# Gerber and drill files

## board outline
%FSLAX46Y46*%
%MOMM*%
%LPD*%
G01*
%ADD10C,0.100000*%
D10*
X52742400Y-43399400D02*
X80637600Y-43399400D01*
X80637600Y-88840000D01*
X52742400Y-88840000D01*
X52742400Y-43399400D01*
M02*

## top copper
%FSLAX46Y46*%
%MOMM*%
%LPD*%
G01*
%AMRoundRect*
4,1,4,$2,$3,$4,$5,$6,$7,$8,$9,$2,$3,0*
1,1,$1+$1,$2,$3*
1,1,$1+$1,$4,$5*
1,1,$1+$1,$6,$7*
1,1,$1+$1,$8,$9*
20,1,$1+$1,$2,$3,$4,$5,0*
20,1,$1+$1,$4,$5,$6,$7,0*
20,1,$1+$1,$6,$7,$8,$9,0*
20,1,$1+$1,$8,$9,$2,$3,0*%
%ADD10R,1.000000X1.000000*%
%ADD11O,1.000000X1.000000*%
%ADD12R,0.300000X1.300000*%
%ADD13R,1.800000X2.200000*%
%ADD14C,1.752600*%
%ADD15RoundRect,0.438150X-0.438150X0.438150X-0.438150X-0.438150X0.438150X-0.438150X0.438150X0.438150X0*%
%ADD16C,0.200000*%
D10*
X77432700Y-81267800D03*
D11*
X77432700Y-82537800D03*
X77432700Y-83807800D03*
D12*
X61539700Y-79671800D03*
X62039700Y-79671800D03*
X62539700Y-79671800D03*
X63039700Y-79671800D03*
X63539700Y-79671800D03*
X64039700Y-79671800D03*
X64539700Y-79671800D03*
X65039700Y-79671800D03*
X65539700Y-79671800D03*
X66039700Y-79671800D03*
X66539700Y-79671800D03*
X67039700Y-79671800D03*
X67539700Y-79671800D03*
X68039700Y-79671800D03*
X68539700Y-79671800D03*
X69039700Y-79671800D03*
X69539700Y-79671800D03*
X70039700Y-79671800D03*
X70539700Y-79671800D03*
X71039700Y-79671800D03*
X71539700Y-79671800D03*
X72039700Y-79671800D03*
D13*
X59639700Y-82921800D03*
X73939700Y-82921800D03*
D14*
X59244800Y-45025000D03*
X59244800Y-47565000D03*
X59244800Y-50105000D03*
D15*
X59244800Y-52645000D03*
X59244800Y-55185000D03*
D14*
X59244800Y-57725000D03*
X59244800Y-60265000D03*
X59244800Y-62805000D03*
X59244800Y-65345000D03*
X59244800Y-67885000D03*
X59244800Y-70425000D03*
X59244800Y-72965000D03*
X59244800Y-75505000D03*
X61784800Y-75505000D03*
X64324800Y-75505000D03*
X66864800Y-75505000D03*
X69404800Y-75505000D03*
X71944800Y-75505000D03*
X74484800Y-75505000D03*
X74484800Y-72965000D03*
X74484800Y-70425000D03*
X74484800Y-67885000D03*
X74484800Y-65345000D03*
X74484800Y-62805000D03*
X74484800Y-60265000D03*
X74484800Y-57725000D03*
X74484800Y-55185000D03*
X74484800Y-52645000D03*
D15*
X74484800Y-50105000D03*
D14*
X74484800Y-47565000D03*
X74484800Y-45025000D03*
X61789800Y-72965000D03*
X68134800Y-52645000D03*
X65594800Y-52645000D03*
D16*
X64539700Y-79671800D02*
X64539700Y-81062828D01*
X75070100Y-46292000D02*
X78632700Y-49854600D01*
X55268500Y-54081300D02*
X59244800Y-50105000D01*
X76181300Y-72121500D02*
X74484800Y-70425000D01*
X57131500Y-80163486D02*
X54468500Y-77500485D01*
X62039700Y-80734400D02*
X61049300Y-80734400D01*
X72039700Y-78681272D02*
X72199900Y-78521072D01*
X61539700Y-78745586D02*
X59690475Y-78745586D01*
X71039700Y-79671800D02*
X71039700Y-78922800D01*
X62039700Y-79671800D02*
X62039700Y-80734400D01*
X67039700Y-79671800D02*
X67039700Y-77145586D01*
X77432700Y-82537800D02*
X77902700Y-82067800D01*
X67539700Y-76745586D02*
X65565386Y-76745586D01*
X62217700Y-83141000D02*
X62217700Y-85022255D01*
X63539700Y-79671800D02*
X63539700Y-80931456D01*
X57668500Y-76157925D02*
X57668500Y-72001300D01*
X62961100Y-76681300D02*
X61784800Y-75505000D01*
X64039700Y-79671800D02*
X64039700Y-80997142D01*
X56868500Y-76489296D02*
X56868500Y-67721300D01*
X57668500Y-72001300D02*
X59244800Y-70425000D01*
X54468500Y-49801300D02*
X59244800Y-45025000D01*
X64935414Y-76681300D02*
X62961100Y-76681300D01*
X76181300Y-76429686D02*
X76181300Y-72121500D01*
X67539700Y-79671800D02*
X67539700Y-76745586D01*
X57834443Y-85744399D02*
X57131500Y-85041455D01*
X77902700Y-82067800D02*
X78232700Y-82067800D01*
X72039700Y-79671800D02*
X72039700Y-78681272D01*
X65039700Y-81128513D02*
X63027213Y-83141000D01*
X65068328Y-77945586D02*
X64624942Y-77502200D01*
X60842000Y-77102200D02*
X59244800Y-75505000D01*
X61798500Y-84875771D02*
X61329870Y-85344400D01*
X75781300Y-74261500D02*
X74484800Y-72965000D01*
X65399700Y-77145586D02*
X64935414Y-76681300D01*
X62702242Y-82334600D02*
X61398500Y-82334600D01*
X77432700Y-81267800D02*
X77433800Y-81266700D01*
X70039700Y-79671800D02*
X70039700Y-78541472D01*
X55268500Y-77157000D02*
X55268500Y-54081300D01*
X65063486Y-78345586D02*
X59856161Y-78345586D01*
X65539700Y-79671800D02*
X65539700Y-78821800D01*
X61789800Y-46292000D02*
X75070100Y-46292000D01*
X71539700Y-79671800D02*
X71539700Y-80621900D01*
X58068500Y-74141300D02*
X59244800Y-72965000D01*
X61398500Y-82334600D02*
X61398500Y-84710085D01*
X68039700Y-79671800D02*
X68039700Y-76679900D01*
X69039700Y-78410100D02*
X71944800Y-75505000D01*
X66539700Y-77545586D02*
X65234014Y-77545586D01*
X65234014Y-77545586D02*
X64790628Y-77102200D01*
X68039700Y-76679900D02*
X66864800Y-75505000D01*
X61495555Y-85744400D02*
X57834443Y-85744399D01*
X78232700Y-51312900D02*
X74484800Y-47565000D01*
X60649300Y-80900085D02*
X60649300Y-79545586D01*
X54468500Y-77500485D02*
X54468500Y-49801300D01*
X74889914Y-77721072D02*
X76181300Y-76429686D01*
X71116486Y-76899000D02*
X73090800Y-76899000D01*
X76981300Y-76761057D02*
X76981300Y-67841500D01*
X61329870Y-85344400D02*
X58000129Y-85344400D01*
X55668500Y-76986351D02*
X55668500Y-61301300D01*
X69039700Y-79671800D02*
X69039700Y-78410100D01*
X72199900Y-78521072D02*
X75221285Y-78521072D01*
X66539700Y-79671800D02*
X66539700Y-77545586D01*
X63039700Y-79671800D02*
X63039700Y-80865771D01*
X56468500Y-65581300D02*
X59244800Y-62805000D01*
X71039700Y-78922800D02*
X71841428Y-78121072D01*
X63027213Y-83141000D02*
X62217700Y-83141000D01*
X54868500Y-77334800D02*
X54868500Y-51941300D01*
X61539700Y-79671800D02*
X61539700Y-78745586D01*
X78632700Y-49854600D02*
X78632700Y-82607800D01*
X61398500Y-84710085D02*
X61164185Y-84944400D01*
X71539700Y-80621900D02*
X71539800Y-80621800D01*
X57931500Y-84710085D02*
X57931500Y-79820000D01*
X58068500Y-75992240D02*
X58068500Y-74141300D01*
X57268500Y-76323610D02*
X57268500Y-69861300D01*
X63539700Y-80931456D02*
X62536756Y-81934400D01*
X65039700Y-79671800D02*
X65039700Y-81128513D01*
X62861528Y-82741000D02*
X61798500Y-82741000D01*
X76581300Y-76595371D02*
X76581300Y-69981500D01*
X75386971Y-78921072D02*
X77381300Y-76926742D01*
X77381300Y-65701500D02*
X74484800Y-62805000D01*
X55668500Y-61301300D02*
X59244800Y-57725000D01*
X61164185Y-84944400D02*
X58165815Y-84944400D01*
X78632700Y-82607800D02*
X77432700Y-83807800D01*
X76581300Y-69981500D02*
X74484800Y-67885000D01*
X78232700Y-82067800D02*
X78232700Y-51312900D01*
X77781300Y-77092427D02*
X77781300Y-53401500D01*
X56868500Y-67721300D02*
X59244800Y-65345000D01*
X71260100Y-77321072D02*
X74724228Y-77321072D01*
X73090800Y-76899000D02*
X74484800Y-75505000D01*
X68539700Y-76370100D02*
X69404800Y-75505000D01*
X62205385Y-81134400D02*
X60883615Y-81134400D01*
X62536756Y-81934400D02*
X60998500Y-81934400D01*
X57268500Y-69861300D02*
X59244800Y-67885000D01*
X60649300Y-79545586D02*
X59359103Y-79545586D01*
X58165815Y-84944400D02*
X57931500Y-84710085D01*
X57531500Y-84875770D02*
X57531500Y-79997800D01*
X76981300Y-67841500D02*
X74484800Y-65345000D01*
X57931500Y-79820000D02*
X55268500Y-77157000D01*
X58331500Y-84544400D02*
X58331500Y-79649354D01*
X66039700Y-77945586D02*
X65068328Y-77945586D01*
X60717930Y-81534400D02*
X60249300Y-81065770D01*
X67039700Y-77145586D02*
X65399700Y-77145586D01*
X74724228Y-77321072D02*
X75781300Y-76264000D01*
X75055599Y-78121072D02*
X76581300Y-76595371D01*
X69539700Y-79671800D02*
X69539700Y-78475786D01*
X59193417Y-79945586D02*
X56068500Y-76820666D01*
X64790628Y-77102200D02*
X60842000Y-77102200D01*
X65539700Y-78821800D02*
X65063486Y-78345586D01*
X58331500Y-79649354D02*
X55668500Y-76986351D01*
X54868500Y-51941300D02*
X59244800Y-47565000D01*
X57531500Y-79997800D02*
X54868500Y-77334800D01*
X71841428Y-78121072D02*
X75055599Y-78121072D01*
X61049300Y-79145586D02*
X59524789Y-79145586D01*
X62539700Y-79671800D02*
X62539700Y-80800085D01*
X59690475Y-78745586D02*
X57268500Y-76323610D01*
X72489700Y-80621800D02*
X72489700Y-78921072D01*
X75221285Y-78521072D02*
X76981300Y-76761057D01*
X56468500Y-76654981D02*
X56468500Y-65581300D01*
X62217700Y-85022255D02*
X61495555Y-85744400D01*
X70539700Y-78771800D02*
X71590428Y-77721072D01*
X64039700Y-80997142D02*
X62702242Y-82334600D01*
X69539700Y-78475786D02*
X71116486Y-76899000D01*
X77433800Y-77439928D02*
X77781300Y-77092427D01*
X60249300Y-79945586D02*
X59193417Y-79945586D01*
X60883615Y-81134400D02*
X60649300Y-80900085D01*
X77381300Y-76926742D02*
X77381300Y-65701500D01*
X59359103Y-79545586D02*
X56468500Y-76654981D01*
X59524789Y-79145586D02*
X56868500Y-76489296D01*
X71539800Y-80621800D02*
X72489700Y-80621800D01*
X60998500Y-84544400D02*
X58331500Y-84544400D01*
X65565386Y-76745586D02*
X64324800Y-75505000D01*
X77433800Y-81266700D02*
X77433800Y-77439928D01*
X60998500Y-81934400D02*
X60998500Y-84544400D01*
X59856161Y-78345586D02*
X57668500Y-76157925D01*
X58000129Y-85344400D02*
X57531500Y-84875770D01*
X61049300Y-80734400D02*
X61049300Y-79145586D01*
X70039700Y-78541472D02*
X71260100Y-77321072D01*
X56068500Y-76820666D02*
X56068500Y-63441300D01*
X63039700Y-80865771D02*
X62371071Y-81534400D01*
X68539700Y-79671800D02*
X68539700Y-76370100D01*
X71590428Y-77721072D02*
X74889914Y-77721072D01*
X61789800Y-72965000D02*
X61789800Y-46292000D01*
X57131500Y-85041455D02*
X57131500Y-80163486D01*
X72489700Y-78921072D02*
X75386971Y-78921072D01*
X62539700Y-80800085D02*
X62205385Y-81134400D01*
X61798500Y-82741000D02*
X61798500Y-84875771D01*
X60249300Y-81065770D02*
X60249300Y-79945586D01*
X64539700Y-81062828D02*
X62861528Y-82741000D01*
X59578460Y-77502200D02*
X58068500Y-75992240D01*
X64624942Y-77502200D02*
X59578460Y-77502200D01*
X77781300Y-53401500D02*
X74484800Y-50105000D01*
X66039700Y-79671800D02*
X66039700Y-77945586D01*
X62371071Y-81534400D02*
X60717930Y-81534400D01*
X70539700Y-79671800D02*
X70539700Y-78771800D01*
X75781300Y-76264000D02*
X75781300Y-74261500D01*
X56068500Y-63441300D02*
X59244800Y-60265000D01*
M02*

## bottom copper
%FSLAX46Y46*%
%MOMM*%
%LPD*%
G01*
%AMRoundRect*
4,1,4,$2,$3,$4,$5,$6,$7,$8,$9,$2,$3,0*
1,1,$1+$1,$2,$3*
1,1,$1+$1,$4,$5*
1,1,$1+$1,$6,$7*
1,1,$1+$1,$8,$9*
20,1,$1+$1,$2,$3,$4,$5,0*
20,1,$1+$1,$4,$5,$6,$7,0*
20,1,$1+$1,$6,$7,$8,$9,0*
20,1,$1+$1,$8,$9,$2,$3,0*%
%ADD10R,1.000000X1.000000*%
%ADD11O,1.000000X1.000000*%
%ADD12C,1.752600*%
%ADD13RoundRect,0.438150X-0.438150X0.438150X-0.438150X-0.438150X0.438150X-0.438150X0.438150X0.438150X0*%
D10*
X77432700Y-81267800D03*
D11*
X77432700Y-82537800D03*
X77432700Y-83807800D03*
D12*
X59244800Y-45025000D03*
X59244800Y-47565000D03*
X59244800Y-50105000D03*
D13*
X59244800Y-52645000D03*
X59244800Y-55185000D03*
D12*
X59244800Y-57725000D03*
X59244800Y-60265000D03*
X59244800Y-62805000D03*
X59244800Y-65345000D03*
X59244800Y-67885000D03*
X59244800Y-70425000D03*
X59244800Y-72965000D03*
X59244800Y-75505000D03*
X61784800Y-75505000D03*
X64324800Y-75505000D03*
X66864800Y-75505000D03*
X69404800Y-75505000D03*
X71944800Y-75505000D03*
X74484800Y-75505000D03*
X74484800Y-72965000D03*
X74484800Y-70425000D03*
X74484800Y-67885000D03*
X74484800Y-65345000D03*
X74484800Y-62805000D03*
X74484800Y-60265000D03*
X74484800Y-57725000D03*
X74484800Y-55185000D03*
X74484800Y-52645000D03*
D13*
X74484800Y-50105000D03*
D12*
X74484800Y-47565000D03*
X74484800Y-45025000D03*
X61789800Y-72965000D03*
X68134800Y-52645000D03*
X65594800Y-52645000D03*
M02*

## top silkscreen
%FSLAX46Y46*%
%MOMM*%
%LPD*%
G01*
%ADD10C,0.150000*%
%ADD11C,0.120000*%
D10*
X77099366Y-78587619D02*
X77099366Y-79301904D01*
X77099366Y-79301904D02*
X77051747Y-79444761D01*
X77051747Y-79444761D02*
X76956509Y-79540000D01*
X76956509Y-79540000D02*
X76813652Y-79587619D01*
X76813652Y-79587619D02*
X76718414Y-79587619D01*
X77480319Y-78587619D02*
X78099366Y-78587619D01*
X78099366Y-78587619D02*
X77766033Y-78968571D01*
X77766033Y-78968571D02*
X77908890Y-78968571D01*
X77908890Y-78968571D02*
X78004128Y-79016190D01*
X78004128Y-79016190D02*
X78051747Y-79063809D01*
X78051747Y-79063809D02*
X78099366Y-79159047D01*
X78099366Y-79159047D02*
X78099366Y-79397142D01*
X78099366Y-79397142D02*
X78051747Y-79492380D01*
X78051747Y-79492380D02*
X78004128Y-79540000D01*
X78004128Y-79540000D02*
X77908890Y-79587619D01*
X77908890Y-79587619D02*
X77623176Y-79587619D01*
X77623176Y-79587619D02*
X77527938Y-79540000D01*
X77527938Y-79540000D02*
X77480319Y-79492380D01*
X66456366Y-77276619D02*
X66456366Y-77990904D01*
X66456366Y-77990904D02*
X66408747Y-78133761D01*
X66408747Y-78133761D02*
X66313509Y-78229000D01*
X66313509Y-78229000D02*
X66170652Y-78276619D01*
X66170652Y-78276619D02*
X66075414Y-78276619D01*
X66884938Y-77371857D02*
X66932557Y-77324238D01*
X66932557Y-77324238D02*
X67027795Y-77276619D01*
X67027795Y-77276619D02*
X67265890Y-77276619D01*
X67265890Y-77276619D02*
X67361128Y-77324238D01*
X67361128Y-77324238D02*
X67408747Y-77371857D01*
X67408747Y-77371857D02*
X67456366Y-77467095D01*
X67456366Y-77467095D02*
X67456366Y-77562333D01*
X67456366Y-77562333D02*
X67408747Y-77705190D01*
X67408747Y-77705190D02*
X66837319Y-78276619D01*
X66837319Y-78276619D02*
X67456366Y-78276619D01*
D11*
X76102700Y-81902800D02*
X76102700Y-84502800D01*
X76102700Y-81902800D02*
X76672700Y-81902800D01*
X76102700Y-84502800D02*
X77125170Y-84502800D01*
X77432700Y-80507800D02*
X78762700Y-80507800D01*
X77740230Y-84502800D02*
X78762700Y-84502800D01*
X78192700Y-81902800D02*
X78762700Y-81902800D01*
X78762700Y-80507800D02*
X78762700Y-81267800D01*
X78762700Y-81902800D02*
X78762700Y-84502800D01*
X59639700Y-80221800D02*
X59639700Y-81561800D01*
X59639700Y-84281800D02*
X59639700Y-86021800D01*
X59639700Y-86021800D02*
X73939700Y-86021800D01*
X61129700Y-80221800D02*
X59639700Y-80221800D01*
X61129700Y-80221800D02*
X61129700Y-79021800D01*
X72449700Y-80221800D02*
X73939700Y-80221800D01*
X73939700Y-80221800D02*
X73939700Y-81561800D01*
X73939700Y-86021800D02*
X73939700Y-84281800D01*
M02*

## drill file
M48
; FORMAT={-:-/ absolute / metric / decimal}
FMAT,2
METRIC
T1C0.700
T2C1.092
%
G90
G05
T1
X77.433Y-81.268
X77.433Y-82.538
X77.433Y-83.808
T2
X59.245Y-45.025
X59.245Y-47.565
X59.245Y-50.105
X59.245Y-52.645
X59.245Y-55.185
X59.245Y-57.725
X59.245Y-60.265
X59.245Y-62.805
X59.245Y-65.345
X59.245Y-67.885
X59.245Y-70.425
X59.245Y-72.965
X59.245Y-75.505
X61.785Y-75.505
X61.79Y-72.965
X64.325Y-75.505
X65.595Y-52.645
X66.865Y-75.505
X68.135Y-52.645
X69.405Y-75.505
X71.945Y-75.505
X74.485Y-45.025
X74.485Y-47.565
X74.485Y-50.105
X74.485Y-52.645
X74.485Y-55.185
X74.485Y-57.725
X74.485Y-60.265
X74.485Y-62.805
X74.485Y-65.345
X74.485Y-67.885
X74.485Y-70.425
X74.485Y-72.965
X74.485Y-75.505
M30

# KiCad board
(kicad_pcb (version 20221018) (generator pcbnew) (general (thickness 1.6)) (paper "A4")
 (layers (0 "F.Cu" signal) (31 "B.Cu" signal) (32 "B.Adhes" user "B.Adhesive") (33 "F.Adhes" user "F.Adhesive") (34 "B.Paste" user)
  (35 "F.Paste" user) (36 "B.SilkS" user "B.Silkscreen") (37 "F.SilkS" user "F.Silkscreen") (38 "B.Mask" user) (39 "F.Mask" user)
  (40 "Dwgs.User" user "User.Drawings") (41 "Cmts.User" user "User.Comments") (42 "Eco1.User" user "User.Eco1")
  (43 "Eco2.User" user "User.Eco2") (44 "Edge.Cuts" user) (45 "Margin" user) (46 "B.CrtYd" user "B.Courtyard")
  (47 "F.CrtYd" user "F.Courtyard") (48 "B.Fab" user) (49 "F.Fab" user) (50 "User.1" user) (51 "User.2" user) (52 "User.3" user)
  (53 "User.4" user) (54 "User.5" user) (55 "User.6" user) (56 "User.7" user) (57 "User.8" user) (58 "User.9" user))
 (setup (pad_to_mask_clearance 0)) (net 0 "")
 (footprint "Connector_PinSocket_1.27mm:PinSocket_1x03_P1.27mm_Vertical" (layer "F.Cu") (at 77.4327 81.2678)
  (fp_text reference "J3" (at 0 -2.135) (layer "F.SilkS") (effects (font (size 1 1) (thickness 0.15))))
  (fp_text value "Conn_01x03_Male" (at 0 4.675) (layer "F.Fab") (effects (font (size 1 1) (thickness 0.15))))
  (fp_line (start -1.33 0.635) (end -1.33 3.235) (stroke (width 0.12) (type solid)) (layer "F.SilkS"))
  (fp_line (start -1.33 0.635) (end -0.76 0.635) (stroke (width 0.12) (type solid)) (layer "F.SilkS"))
  (fp_line (start -1.33 3.235) (end -0.30753 3.235) (stroke (width 0.12) (type solid)) (layer "F.SilkS"))
  (fp_line (start 0 -0.76) (end 1.33 -0.76) (stroke (width 0.12) (type solid)) (layer "F.SilkS"))
  (fp_line (start 0.30753 3.235) (end 1.33 3.235) (stroke (width 0.12) (type solid)) (layer "F.SilkS"))
  (fp_line (start 0.76 0.635) (end 1.33 0.635) (stroke (width 0.12) (type solid)) (layer "F.SilkS"))
  (fp_line (start 1.33 -0.76) (end 1.33 0) (stroke (width 0.12) (type solid)) (layer "F.SilkS"))
  (fp_line (start 1.33 0.635) (end 1.33 3.235) (stroke (width 0.12) (type solid)) (layer "F.SilkS"))
  (pad "1" thru_hole rect (at 0 0) (size 1 1) (drill 0.7) (layers "*.Cu" "*.Mask"))
  (pad "2" thru_hole oval (at 0 1.27) (size 1 1) (drill 0.7) (layers "*.Cu" "*.Mask"))
  (pad "3" thru_hole oval (at 0 2.54) (size 1 1) (drill 0.7) (layers "*.Cu" "*.Mask")))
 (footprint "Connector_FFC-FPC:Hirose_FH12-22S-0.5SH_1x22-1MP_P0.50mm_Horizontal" (layer "F.Cu") (at 66.7897 81.5218)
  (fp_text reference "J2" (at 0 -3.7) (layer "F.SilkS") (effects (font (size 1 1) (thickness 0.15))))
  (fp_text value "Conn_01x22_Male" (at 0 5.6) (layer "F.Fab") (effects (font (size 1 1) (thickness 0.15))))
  (fp_line (start -7.15 -1.3) (end -7.15 0.04) (stroke (width 0.12) (type solid)) (layer "F.SilkS"))
  (fp_line (start -7.15 2.76) (end -7.15 4.5) (stroke (width 0.12) (type solid)) (layer "F.SilkS"))
  (fp_line (start -7.15 4.5) (end 7.15 4.5) (stroke (width 0.12) (type solid)) (layer "F.SilkS"))
  (fp_line (start -5.66 -1.3) (end -7.15 -1.3) (stroke (width 0.12) (type solid)) (layer "F.SilkS"))
  (fp_line (start -5.66 -1.3) (end -5.66 -2.5) (stroke (width 0.12) (type solid)) (layer "F.SilkS"))
  (fp_line (start 5.66 -1.3) (end 7.15 -1.3) (stroke (width 0.12) (type solid)) (layer "F.SilkS"))
  (fp_line (start 7.15 -1.3) (end 7.15 0.04) (stroke (width 0.12) (type solid)) (layer "F.SilkS"))
  (fp_line (start 7.15 4.5) (end 7.15 2.76) (stroke (width 0.12) (type solid)) (layer "F.SilkS"))
  (pad "1" smd rect (at -5.25 -1.85) (size 0.3 1.3) (layers "F.Cu" "F.Paste" "F.Mask"))
  (pad "2" smd rect (at -4.75 -1.85) (size 0.3 1.3) (layers "F.Cu" "F.Paste" "F.Mask"))
  (pad "3" smd rect (at -4.25 -1.85) (size 0.3 1.3) (layers "F.Cu" "F.Paste" "F.Mask"))
  (pad "4" smd rect (at -3.75 -1.85) (size 0.3 1.3) (layers "F.Cu" "F.Paste" "F.Mask"))
  (pad "5" smd rect (at -3.25 -1.85) (size 0.3 1.3) (layers "F.Cu" "F.Paste" "F.Mask"))
  (pad "6" smd rect (at -2.75 -1.85) (size 0.3 1.3) (layers "F.Cu" "F.Paste" "F.Mask"))
  (pad "7" smd rect (at -2.25 -1.85) (size 0.3 1.3) (layers "F.Cu" "F.Paste" "F.Mask"))
  (pad "8" smd rect (at -1.75 -1.85) (size 0.3 1.3) (layers "F.Cu" "F.Paste" "F.Mask"))
  (pad "9" smd rect (at -1.25 -1.85) (size 0.3 1.3) (layers "F.Cu" "F.Paste" "F.Mask"))
  (pad "10" smd rect (at -0.75 -1.85) (size 0.3 1.3) (layers "F.Cu" "F.Paste" "F.Mask"))
  (pad "11" smd rect (at -0.25 -1.85) (size 0.3 1.3) (layers "F.Cu" "F.Paste" "F.Mask"))
  (pad "12" smd rect (at 0.25 -1.85) (size 0.3 1.3) (layers "F.Cu" "F.Paste" "F.Mask"))
  (pad "13" smd rect (at 0.75 -1.85) (size 0.3 1.3) (layers "F.Cu" "F.Paste" "F.Mask"))
  (pad "14" smd rect (at 1.25 -1.85) (size 0.3 1.3) (layers "F.Cu" "F.Paste" "F.Mask"))
  (pad "15" smd rect (at 1.75 -1.85) (size 0.3 1.3) (layers "F.Cu" "F.Paste" "F.Mask"))
  (pad "16" smd rect (at 2.25 -1.85) (size 0.3 1.3) (layers "F.Cu" "F.Paste" "F.Mask"))
  (pad "17" smd rect (at 2.75 -1.85) (size 0.3 1.3) (layers "F.Cu" "F.Paste" "F.Mask"))
  (pad "18" smd rect (at 3.25 -1.85) (size 0.3 1.3) (layers "F.Cu" "F.Paste" "F.Mask"))
  (pad "19" smd rect (at 3.75 -1.85) (size 0.3 1.3) (layers "F.Cu" "F.Paste" "F.Mask"))
  (pad "20" smd rect (at 4.25 -1.85) (size 0.3 1.3) (layers "F.Cu" "F.Paste" "F.Mask"))
  (pad "21" smd rect (at 4.75 -1.85) (size 0.3 1.3) (layers "F.Cu" "F.Paste" "F.Mask"))
  (pad "22" smd rect (at 5.25 -1.85) (size 0.3 1.3) (layers "F.Cu" "F.Paste" "F.Mask"))
  (pad "MP" smd rect (at -7.15 1.4) (size 1.8 2.2) (layers "F.Cu" "F.Paste" "F.Mask"))
  (pad "MP" smd rect (at 7.15 1.4) (size 1.8 2.2) (layers "F.Cu" "F.Paste" "F.Mask")))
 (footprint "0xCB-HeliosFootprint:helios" (layer "F.Cu") (at 66.8648 61.535)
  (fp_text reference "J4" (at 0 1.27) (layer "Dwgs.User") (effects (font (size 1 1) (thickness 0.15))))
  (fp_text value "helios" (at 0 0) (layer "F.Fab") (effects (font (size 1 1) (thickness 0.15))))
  (pad "1" thru_hole circle (at -7.62 -16.51 270) (size 1.7526 1.7526) (drill 1.0922) (layers "*.Cu" "*.Mask"))
  (pad "2" thru_hole circle (at -7.62 -13.97 270) (size 1.7526 1.7526) (drill 1.0922) (layers "*.Cu" "*.Mask"))
  (pad "3" thru_hole circle (at -7.62 -11.43 270) (size 1.7526 1.7526) (drill 1.0922) (layers "*.Cu" "*.Mask"))
  (pad "4" thru_hole roundrect (at -7.62 -8.89 270) (size 1.7526 1.7526) (drill 1.0922) (layers "*.Cu" "*.Mask") (roundrect_rratio 0.25))
  (pad "5" thru_hole roundrect (at -7.62 -6.35 270) (size 1.7526 1.7526) (drill 1.0922) (layers "*.Cu" "*.Mask") (roundrect_rratio 0.25))
  (pad "6" thru_hole circle (at -7.62 -3.81 270) (size 1.7526 1.7526) (drill 1.0922) (layers "*.Cu" "*.Mask"))
  (pad "7" thru_hole circle (at -7.62 -1.27 270) (size 1.7526 1.7526) (drill 1.0922) (layers "*.Cu" "*.Mask"))
  (pad "8" thru_hole circle (at -7.62 1.27 270) (size 1.7526 1.7526) (drill 1.0922) (layers "*.Cu" "*.Mask"))
  (pad "9" thru_hole circle (at -7.62 3.81 270) (size 1.7526 1.7526) (drill 1.0922) (layers "*.Cu" "*.Mask"))
  (pad "10" thru_hole circle (at -7.62 6.35 270) (size 1.7526 1.7526) (drill 1.0922) (layers "*.Cu" "*.Mask"))
  (pad "11" thru_hole circle (at -7.62 8.89 270) (size 1.7526 1.7526) (drill 1.0922) (layers "*.Cu" "*.Mask"))
  (pad "12" thru_hole circle (at -7.62 11.43 270) (size 1.7526 1.7526) (drill 1.0922) (layers "*.Cu" "*.Mask"))
  (pad "13" thru_hole circle (at -7.62 13.97 270) (size 1.7526 1.7526) (drill 1.0922) (layers "*.Cu" "*.Mask"))
  (pad "14" thru_hole circle (at -5.08 13.97 270) (size 1.7526 1.7526) (drill 1.0922) (layers "*.Cu" "*.Mask"))
  (pad "15" thru_hole circle (at -2.54 13.97 270) (size 1.7526 1.7526) (drill 1.0922) (layers "*.Cu" "*.Mask"))
  (pad "16" thru_hole circle (at 0 13.97 270) (size 1.7526 1.7526) (drill 1.0922) (layers "*.Cu" "*.Mask"))
  (pad "17" thru_hole circle (at 2.54 13.97 270) (size 1.7526 1.7526) (drill 1.0922) (layers "*.Cu" "*.Mask"))
  (pad "18" thru_hole circle (at 5.08 13.97 270) (size 1.7526 1.7526) (drill 1.0922) (layers "*.Cu" "*.Mask"))
  (pad "19" thru_hole circle (at 7.62 13.97 270) (size 1.7526 1.7526) (drill 1.0922) (layers "*.Cu" "*.Mask"))
  (pad "20" thru_hole circle (at 7.62 11.43 270) (size 1.7526 1.7526) (drill 1.0922) (layers "*.Cu" "*.Mask"))
  (pad "21" thru_hole circle (at 7.62 8.89 270) (size 1.7526 1.7526) (drill 1.0922) (layers "*.Cu" "*.Mask"))
  (pad "22" thru_hole circle (at 7.62 6.35 270) (size 1.7526 1.7526) (drill 1.0922) (layers "*.Cu" "*.Mask"))
  (pad "23" thru_hole circle (at 7.62 3.81 270) (size 1.7526 1.7526) (drill 1.0922) (layers "*.Cu" "*.Mask"))
  (pad "24" thru_hole circle (at 7.62 1.27 270) (size 1.7526 1.7526) (drill 1.0922) (layers "*.Cu" "*.Mask"))
  (pad "25" thru_hole circle (at 7.62 -1.27 270) (size 1.7526 1.7526) (drill 1.0922) (layers "*.Cu" "*.Mask"))
  (pad "26" thru_hole circle (at 7.62 -3.81 270) (size 1.7526 1.7526) (drill 1.0922) (layers "*.Cu" "*.Mask"))
  (pad "27" thru_hole circle (at 7.62 -6.35 270) (size 1.7526 1.7526) (drill 1.0922) (layers "*.Cu" "*.Mask"))
  (pad "28" thru_hole circle (at 7.62 -8.89 270) (size 1.7526 1.7526) (drill 1.0922) (layers "*.Cu" "*.Mask"))
  (pad "29" thru_hole roundrect (at 7.62 -11.43 270) (size 1.7526 1.7526) (drill 1.0922) (layers "*.Cu" "*.Mask") (roundrect_rratio 0.25))
  (pad "30" thru_hole circle (at 7.62 -13.97 270) (size 1.7526 1.7526) (drill 1.0922) (layers "*.Cu" "*.Mask"))
  (pad "31" thru_hole circle (at 7.62 -16.51 270) (size 1.7526 1.7526) (drill 1.0922) (layers "*.Cu" "*.Mask"))
  (pad "32" thru_hole circle (at -5.075 11.43 270) (size 1.7526 1.7526) (drill 1.0922) (layers "*.Cu" "*.Mask"))
  (pad "33" thru_hole circle (at 1.27 -8.89 270) (size 1.7526 1.7526) (drill 1.0922) (layers "*.Cu" "*.Mask"))
  (pad "34" thru_hole circle (at -1.27 -8.89 270) (size 1.7526 1.7526) (drill 1.0922) (layers "*.Cu" "*.Mask")))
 (gr_rect (start 52.7424 43.3994) (end 80.6376 88.84) (stroke (width 0.1) (type solid)) (fill none) (layer "Edge.Cuts"))
 (segment (start 64.5397 79.6718) (end 64.5397 81.062828) (width 0.2) (layer "F.Cu") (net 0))
 (segment (start 75.0701 46.292) (end 78.6327 49.8546) (width 0.2) (layer "F.Cu") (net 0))
 (segment (start 55.2685 54.0813) (end 59.2448 50.105) (width 0.2) (layer "F.Cu") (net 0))
 (segment (start 76.1813 72.1215) (end 74.4848 70.425) (width 0.2) (layer "F.Cu") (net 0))
 (segment (start 57.1315 80.163486) (end 54.4685 77.500485) (width 0.2) (layer "F.Cu") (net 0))
 (segment (start 62.0397 80.7344) (end 61.0493 80.7344) (width 0.2) (layer "F.Cu") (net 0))
 (segment (start 72.0397 78.681272) (end 72.1999 78.521072) (width 0.2) (layer "F.Cu") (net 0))
 (segment (start 61.5397 78.745586) (end 59.690475 78.745586) (width 0.2) (layer "F.Cu") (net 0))
 (segment (start 71.0397 79.6718) (end 71.0397 78.9228) (width 0.2) (layer "F.Cu") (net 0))
 (segment (start 62.0397 79.6718) (end 62.0397 80.7344) (width 0.2) (layer "F.Cu") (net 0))
 (segment (start 67.0397 79.6718) (end 67.0397 77.145586) (width 0.2) (layer "F.Cu") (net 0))
 (segment (start 77.4327 82.5378) (end 77.9027 82.0678) (width 0.2) (layer "F.Cu") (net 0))
 (segment (start 67.5397 76.745586) (end 65.565386 76.745586) (width 0.2) (layer "F.Cu") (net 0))
 (segment (start 62.2177 83.141) (end 62.2177 85.022255) (width 0.2) (layer "F.Cu") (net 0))
 (segment (start 63.5397 79.6718) (end 63.5397 80.931456) (width 0.2) (layer "F.Cu") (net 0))
 (segment (start 57.6685 76.157925) (end 57.6685 72.0013) (width 0.2) (layer "F.Cu") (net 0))
 (segment (start 62.9611 76.6813) (end 61.7848 75.505) (width 0.2) (layer "F.Cu") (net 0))
 (segment (start 64.0397 79.6718) (end 64.0397 80.997142) (width 0.2) (layer "F.Cu") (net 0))
 (segment (start 56.8685 76.489296) (end 56.8685 67.7213) (width 0.2) (layer "F.Cu") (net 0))
 (segment (start 57.6685 72.0013) (end 59.2448 70.425) (width 0.2) (layer "F.Cu") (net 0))
 (segment (start 54.4685 49.8013) (end 59.2448 45.025) (width 0.2) (layer "F.Cu") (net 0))
 (segment (start 64.935414 76.6813) (end 62.9611 76.6813) (width 0.2) (layer "F.Cu") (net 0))
 (segment (start 76.1813 76.429686) (end 76.1813 72.1215) (width 0.2) (layer "F.Cu") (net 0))
 (segment (start 67.5397 79.6718) (end 67.5397 76.745586) (width 0.2) (layer "F.Cu") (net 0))
 (segment (start 57.834443 85.744399) (end 57.1315 85.041455) (width 0.2) (layer "F.Cu") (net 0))
 (segment (start 77.9027 82.0678) (end 78.2327 82.0678) (width 0.2) (layer "F.Cu") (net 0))
 (segment (start 72.0397 79.6718) (end 72.0397 78.681272) (width 0.2) (layer "F.Cu") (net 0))
 (segment (start 65.0397 81.128513) (end 63.027213 83.141) (width 0.2) (layer "F.Cu") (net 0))
 (segment (start 65.068328 77.945586) (end 64.624942 77.5022) (width 0.2) (layer "F.Cu") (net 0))
 (segment (start 60.842 77.1022) (end 59.2448 75.505) (width 0.2) (layer "F.Cu") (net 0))
 (segment (start 61.7985 84.875771) (end 61.32987 85.3444) (width 0.2) (layer "F.Cu") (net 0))
 (segment (start 75.7813 74.2615) (end 74.4848 72.965) (width 0.2) (layer "F.Cu") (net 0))
 (segment (start 65.3997 77.145586) (end 64.935414 76.6813) (width 0.2) (layer "F.Cu") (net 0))
 (segment (start 62.702242 82.3346) (end 61.3985 82.3346) (width 0.2) (layer "F.Cu") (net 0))
 (segment (start 77.4327 81.2678) (end 77.4338 81.2667) (width 0.2) (layer "F.Cu") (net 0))
 (segment (start 70.0397 79.6718) (end 70.0397 78.541472) (width 0.2) (layer "F.Cu") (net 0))
 (segment (start 55.2685 77.157) (end 55.2685 54.0813) (width 0.2) (layer "F.Cu") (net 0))
 (segment (start 65.063486 78.345586) (end 59.856161 78.345586) (width 0.2) (layer "F.Cu") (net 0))
 (segment (start 65.5397 79.6718) (end 65.5397 78.8218) (width 0.2) (layer "F.Cu") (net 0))
 (segment (start 61.7898 46.292) (end 75.0701 46.292) (width 0.2) (layer "F.Cu") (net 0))
 (segment (start 71.5397 79.6718) (end 71.5397 80.6219) (width 0.2) (layer "F.Cu") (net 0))
 (segment (start 58.0685 74.1413) (end 59.2448 72.965) (width 0.2) (layer "F.Cu") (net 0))
 (segment (start 61.3985 82.3346) (end 61.3985 84.710085) (width 0.2) (layer "F.Cu") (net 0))
 (segment (start 68.0397 79.6718) (end 68.0397 76.6799) (width 0.2) (layer "F.Cu") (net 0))
 (segment (start 69.0397 78.4101) (end 71.9448 75.505) (width 0.2) (layer "F.Cu") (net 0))
 (segment (start 66.5397 77.545586) (end 65.234014 77.545586) (width 0.2) (layer "F.Cu") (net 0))
 (segment (start 65.234014 77.545586) (end 64.790628 77.1022) (width 0.2) (layer "F.Cu") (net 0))
 (segment (start 68.0397 76.6799) (end 66.8648 75.505) (width 0.2) (layer "F.Cu") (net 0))
 (segment (start 61.495555 85.7444) (end 57.834443 85.744399) (width 0.2) (layer "F.Cu") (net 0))
 (segment (start 78.2327 51.3129) (end 74.4848 47.565) (width 0.2) (layer "F.Cu") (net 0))
 (segment (start 60.6493 80.900085) (end 60.6493 79.545586) (width 0.2) (layer "F.Cu") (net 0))
 (segment (start 54.4685 77.500485) (end 54.4685 49.8013) (width 0.2) (layer "F.Cu") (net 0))
 (segment (start 74.889914 77.721072) (end 76.1813 76.429686) (width 0.2) (layer "F.Cu") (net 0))
 (segment (start 71.116486 76.899) (end 73.0908 76.899) (width 0.2) (layer "F.Cu") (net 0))
 (segment (start 76.9813 76.761057) (end 76.9813 67.8415) (width 0.2) (layer "F.Cu") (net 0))
 (segment (start 61.32987 85.3444) (end 58.000129 85.3444) (width 0.2) (layer "F.Cu") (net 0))
 (segment (start 55.6685 76.986351) (end 55.6685 61.3013) (width 0.2) (layer "F.Cu") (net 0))
 (segment (start 69.0397 79.6718) (end 69.0397 78.4101) (width 0.2) (layer "F.Cu") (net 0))
 (segment (start 72.1999 78.521072) (end 75.221285 78.521072) (width 0.2) (layer "F.Cu") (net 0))
 (segment (start 66.5397 79.6718) (end 66.5397 77.545586) (width 0.2) (layer "F.Cu") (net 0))
 (segment (start 63.0397 79.6718) (end 63.0397 80.865771) (width 0.2) (layer "F.Cu") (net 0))
 (segment (start 56.4685 65.5813) (end 59.2448 62.805) (width 0.2) (layer "F.Cu") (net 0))
 (segment (start 71.0397 78.9228) (end 71.841428 78.121072) (width 0.2) (layer "F.Cu") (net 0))
 (segment (start 63.027213 83.141) (end 62.2177 83.141) (width 0.2) (layer "F.Cu") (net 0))
 (segment (start 54.8685 77.3348) (end 54.8685 51.9413) (width 0.2) (layer "F.Cu") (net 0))
 (segment (start 61.5397 79.6718) (end 61.5397 78.745586) (width 0.2) (layer "F.Cu") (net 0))
 (segment (start 78.6327 49.8546) (end 78.6327 82.6078) (width 0.2) (layer "F.Cu") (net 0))
 (segment (start 61.3985 84.710085) (end 61.164185 84.9444) (width 0.2) (layer "F.Cu") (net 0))
 (segment (start 71.5397 80.6219) (end 71.5398 80.6218) (width 0.2) (layer "F.Cu") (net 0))
 (segment (start 57.9315 84.710085) (end 57.9315 79.82) (width 0.2) (layer "F.Cu") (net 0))
 (segment (start 58.0685 75.99224) (end 58.0685 74.1413) (width 0.2) (layer "F.Cu") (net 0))
 (segment (start 57.2685 76.32361) (end 57.2685 69.8613) (width 0.2) (layer "F.Cu") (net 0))
 (segment (start 63.5397 80.931456) (end 62.536756 81.9344) (width 0.2) (layer "F.Cu") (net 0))
 (segment (start 65.0397 79.6718) (end 65.0397 81.128513) (width 0.2) (layer "F.Cu") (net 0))
 (segment (start 62.861528 82.741) (end 61.7985 82.741) (width 0.2) (layer "F.Cu") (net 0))
 (segment (start 76.5813 76.595371) (end 76.5813 69.9815) (width 0.2) (layer "F.Cu") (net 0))
 (segment (start 75.386971 78.921072) (end 77.3813 76.926742) (width 0.2) (layer "F.Cu") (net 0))
 (segment (start 77.3813 65.7015) (end 74.4848 62.805) (width 0.2) (layer "F.Cu") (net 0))
 (segment (start 55.6685 61.3013) (end 59.2448 57.725) (width 0.2) (layer "F.Cu") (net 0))
 (segment (start 61.164185 84.9444) (end 58.165815 84.9444) (width 0.2) (layer "F.Cu") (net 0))
 (segment (start 78.6327 82.6078) (end 77.4327 83.8078) (width 0.2) (layer "F.Cu") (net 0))
 (segment (start 76.5813 69.9815) (end 74.4848 67.885) (width 0.2) (layer "F.Cu") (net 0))
 (segment (start 78.2327 82.0678) (end 78.2327 51.3129) (width 0.2) (layer "F.Cu") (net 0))
 (segment (start 77.7813 77.092427) (end 77.7813 53.4015) (width 0.2) (layer "F.Cu") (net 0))
 (segment (start 56.8685 67.7213) (end 59.2448 65.345) (width 0.2) (layer "F.Cu") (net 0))
 (segment (start 71.2601 77.321072) (end 74.724228 77.321072) (width 0.2) (layer "F.Cu") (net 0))
 (segment (start 73.0908 76.899) (end 74.4848 75.505) (width 0.2) (layer "F.Cu") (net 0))
 (segment (start 68.5397 76.3701) (end 69.4048 75.505) (width 0.2) (layer "F.Cu") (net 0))
 (segment (start 62.205385 81.1344) (end 60.883615 81.1344) (width 0.2) (layer "F.Cu") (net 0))
 (segment (start 62.536756 81.9344) (end 60.9985 81.9344) (width 0.2) (layer "F.Cu") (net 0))
 (segment (start 57.2685 69.8613) (end 59.2448 67.885) (width 0.2) (layer "F.Cu") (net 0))
 (segment (start 60.6493 79.545586) (end 59.359103 79.545586) (width 0.2) (layer "F.Cu") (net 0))
 (segment (start 58.165815 84.9444) (end 57.9315 84.710085) (width 0.2) (layer "F.Cu") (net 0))
 (segment (start 57.5315 84.87577) (end 57.5315 79.9978) (width 0.2) (layer "F.Cu") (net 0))
 (segment (start 76.9813 67.8415) (end 74.4848 65.345) (width 0.2) (layer "F.Cu") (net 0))
 (segment (start 57.9315 79.82) (end 55.2685 77.157) (width 0.2) (layer "F.Cu") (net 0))
 (segment (start 58.3315 84.5444) (end 58.3315 79.649354) (width 0.2) (layer "F.Cu") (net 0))
 (segment (start 66.0397 77.945586) (end 65.068328 77.945586) (width 0.2) (layer "F.Cu") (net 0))
 (segment (start 60.71793 81.5344) (end 60.2493 81.06577) (width 0.2) (layer "F.Cu") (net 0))
 (segment (start 67.0397 77.145586) (end 65.3997 77.145586) (width 0.2) (layer "F.Cu") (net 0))
 (segment (start 74.724228 77.321072) (end 75.7813 76.264) (width 0.2) (layer "F.Cu") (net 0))
 (segment (start 75.055599 78.121072) (end 76.5813 76.595371) (width 0.2) (layer "F.Cu") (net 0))
 (segment (start 69.5397 79.6718) (end 69.5397 78.475786) (width 0.2) (layer "F.Cu") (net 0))
 (segment (start 59.193417 79.945586) (end 56.0685 76.820666) (width 0.2) (layer "F.Cu") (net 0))
 (segment (start 64.790628 77.1022) (end 60.842 77.1022) (width 0.2) (layer "F.Cu") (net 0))
 (segment (start 65.5397 78.8218) (end 65.063486 78.345586) (width 0.2) (layer "F.Cu") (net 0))
 (segment (start 58.3315 79.649354) (end 55.6685 76.986351) (width 0.2) (layer "F.Cu") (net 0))
 (segment (start 54.8685 51.9413) (end 59.2448 47.565) (width 0.2) (layer "F.Cu") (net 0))
 (segment (start 57.5315 79.9978) (end 54.8685 77.3348) (width 0.2) (layer "F.Cu") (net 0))
 (segment (start 71.841428 78.121072) (end 75.055599 78.121072) (width 0.2) (layer "F.Cu") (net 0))
 (segment (start 61.0493 79.145586) (end 59.524789 79.145586) (width 0.2) (layer "F.Cu") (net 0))
 (segment (start 62.5397 79.6718) (end 62.5397 80.800085) (width 0.2) (layer "F.Cu") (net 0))
 (segment (start 59.690475 78.745586) (end 57.2685 76.32361) (width 0.2) (layer "F.Cu") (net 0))
 (segment (start 72.4897 80.6218) (end 72.4897 78.921072) (width 0.2) (layer "F.Cu") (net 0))
 (segment (start 75.221285 78.521072) (end 76.9813 76.761057) (width 0.2) (layer "F.Cu") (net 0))
 (segment (start 56.4685 76.654981) (end 56.4685 65.5813) (width 0.2) (layer "F.Cu") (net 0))
 (segment (start 62.2177 85.022255) (end 61.495555 85.7444) (width 0.2) (layer "F.Cu") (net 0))
 (segment (start 70.5397 78.7718) (end 71.590428 77.721072) (width 0.2) (layer "F.Cu") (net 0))
 (segment (start 64.0397 80.997142) (end 62.702242 82.3346) (width 0.2) (layer "F.Cu") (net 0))
 (segment (start 69.5397 78.475786) (end 71.116486 76.899) (width 0.2) (layer "F.Cu") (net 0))
 (segment (start 77.4338 77.439928) (end 77.7813 77.092427) (width 0.2) (layer "F.Cu") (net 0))
 (segment (start 60.2493 79.945586) (end 59.193417 79.945586) (width 0.2) (layer "F.Cu") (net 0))
 (segment (start 60.883615 81.1344) (end 60.6493 80.900085) (width 0.2) (layer "F.Cu") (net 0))
 (segment (start 77.3813 76.926742) (end 77.3813 65.7015) (width 0.2) (layer "F.Cu") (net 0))
 (segment (start 59.359103 79.545586) (end 56.4685 76.654981) (width 0.2) (layer "F.Cu") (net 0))
 (segment (start 59.524789 79.145586) (end 56.8685 76.489296) (width 0.2) (layer "F.Cu") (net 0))
 (segment (start 71.5398 80.6218) (end 72.4897 80.6218) (width 0.2) (layer "F.Cu") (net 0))
 (segment (start 60.9985 84.5444) (end 58.3315 84.5444) (width 0.2) (layer "F.Cu") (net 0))
 (segment (start 65.565386 76.745586) (end 64.3248 75.505) (width 0.2) (layer "F.Cu") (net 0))
 (segment (start 77.4338 81.2667) (end 77.4338 77.439928) (width 0.2) (layer "F.Cu") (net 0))
 (segment (start 60.9985 81.9344) (end 60.9985 84.5444) (width 0.2) (layer "F.Cu") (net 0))
 (segment (start 59.856161 78.345586) (end 57.6685 76.157925) (width 0.2) (layer "F.Cu") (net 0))
 (segment (start 58.000129 85.3444) (end 57.5315 84.87577) (width 0.2) (layer "F.Cu") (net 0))
 (segment (start 61.0493 80.7344) (end 61.0493 79.145586) (width 0.2) (layer "F.Cu") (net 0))
 (segment (start 70.0397 78.541472) (end 71.2601 77.321072) (width 0.2) (layer "F.Cu") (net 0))
 (segment (start 56.0685 76.820666) (end 56.0685 63.4413) (width 0.2) (layer "F.Cu") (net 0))
 (segment (start 63.0397 80.865771) (end 62.371071 81.5344) (width 0.2) (layer "F.Cu") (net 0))
 (segment (start 68.5397 79.6718) (end 68.5397 76.3701) (width 0.2) (layer "F.Cu") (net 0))
 (segment (start 71.590428 77.721072) (end 74.889914 77.721072) (width 0.2) (layer "F.Cu") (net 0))
 (segment (start 61.7898 72.965) (end 61.7898 46.292) (width 0.2) (layer "F.Cu") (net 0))
 (segment (start 57.1315 85.041455) (end 57.1315 80.163486) (width 0.2) (layer "F.Cu") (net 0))
 (segment (start 72.4897 78.921072) (end 75.386971 78.921072) (width 0.2) (layer "F.Cu") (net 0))
 (segment (start 62.5397 80.800085) (end 62.205385 81.1344) (width 0.2) (layer "F.Cu") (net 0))
 (segment (start 61.7985 82.741) (end 61.7985 84.875771) (width 0.2) (layer "F.Cu") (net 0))
 (segment (start 60.2493 81.06577) (end 60.2493 79.945586) (width 0.2) (layer "F.Cu") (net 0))
 (segment (start 64.5397 81.062828) (end 62.861528 82.741) (width 0.2) (layer "F.Cu") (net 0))
 (segment (start 59.57846 77.5022) (end 58.0685 75.99224) (width 0.2) (layer "F.Cu") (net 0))
 (segment (start 64.624942 77.5022) (end 59.57846 77.5022) (width 0.2) (layer "F.Cu") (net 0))
 (segment (start 77.7813 53.4015) (end 74.4848 50.105) (width 0.2) (layer "F.Cu") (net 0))
 (segment (start 66.0397 79.6718) (end 66.0397 77.945586) (width 0.2) (layer "F.Cu") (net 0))
 (segment (start 62.371071 81.5344) (end 60.71793 81.5344) (width 0.2) (layer "F.Cu") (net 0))
 (segment (start 70.5397 79.6718) (end 70.5397 78.7718) (width 0.2) (layer "F.Cu") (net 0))
 (segment (start 75.7813 76.264) (end 75.7813 74.2615) (width 0.2) (layer "F.Cu") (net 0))
 (segment (start 56.0685 63.4413) (end 59.2448 60.265) (width 0.2) (layer "F.Cu") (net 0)))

